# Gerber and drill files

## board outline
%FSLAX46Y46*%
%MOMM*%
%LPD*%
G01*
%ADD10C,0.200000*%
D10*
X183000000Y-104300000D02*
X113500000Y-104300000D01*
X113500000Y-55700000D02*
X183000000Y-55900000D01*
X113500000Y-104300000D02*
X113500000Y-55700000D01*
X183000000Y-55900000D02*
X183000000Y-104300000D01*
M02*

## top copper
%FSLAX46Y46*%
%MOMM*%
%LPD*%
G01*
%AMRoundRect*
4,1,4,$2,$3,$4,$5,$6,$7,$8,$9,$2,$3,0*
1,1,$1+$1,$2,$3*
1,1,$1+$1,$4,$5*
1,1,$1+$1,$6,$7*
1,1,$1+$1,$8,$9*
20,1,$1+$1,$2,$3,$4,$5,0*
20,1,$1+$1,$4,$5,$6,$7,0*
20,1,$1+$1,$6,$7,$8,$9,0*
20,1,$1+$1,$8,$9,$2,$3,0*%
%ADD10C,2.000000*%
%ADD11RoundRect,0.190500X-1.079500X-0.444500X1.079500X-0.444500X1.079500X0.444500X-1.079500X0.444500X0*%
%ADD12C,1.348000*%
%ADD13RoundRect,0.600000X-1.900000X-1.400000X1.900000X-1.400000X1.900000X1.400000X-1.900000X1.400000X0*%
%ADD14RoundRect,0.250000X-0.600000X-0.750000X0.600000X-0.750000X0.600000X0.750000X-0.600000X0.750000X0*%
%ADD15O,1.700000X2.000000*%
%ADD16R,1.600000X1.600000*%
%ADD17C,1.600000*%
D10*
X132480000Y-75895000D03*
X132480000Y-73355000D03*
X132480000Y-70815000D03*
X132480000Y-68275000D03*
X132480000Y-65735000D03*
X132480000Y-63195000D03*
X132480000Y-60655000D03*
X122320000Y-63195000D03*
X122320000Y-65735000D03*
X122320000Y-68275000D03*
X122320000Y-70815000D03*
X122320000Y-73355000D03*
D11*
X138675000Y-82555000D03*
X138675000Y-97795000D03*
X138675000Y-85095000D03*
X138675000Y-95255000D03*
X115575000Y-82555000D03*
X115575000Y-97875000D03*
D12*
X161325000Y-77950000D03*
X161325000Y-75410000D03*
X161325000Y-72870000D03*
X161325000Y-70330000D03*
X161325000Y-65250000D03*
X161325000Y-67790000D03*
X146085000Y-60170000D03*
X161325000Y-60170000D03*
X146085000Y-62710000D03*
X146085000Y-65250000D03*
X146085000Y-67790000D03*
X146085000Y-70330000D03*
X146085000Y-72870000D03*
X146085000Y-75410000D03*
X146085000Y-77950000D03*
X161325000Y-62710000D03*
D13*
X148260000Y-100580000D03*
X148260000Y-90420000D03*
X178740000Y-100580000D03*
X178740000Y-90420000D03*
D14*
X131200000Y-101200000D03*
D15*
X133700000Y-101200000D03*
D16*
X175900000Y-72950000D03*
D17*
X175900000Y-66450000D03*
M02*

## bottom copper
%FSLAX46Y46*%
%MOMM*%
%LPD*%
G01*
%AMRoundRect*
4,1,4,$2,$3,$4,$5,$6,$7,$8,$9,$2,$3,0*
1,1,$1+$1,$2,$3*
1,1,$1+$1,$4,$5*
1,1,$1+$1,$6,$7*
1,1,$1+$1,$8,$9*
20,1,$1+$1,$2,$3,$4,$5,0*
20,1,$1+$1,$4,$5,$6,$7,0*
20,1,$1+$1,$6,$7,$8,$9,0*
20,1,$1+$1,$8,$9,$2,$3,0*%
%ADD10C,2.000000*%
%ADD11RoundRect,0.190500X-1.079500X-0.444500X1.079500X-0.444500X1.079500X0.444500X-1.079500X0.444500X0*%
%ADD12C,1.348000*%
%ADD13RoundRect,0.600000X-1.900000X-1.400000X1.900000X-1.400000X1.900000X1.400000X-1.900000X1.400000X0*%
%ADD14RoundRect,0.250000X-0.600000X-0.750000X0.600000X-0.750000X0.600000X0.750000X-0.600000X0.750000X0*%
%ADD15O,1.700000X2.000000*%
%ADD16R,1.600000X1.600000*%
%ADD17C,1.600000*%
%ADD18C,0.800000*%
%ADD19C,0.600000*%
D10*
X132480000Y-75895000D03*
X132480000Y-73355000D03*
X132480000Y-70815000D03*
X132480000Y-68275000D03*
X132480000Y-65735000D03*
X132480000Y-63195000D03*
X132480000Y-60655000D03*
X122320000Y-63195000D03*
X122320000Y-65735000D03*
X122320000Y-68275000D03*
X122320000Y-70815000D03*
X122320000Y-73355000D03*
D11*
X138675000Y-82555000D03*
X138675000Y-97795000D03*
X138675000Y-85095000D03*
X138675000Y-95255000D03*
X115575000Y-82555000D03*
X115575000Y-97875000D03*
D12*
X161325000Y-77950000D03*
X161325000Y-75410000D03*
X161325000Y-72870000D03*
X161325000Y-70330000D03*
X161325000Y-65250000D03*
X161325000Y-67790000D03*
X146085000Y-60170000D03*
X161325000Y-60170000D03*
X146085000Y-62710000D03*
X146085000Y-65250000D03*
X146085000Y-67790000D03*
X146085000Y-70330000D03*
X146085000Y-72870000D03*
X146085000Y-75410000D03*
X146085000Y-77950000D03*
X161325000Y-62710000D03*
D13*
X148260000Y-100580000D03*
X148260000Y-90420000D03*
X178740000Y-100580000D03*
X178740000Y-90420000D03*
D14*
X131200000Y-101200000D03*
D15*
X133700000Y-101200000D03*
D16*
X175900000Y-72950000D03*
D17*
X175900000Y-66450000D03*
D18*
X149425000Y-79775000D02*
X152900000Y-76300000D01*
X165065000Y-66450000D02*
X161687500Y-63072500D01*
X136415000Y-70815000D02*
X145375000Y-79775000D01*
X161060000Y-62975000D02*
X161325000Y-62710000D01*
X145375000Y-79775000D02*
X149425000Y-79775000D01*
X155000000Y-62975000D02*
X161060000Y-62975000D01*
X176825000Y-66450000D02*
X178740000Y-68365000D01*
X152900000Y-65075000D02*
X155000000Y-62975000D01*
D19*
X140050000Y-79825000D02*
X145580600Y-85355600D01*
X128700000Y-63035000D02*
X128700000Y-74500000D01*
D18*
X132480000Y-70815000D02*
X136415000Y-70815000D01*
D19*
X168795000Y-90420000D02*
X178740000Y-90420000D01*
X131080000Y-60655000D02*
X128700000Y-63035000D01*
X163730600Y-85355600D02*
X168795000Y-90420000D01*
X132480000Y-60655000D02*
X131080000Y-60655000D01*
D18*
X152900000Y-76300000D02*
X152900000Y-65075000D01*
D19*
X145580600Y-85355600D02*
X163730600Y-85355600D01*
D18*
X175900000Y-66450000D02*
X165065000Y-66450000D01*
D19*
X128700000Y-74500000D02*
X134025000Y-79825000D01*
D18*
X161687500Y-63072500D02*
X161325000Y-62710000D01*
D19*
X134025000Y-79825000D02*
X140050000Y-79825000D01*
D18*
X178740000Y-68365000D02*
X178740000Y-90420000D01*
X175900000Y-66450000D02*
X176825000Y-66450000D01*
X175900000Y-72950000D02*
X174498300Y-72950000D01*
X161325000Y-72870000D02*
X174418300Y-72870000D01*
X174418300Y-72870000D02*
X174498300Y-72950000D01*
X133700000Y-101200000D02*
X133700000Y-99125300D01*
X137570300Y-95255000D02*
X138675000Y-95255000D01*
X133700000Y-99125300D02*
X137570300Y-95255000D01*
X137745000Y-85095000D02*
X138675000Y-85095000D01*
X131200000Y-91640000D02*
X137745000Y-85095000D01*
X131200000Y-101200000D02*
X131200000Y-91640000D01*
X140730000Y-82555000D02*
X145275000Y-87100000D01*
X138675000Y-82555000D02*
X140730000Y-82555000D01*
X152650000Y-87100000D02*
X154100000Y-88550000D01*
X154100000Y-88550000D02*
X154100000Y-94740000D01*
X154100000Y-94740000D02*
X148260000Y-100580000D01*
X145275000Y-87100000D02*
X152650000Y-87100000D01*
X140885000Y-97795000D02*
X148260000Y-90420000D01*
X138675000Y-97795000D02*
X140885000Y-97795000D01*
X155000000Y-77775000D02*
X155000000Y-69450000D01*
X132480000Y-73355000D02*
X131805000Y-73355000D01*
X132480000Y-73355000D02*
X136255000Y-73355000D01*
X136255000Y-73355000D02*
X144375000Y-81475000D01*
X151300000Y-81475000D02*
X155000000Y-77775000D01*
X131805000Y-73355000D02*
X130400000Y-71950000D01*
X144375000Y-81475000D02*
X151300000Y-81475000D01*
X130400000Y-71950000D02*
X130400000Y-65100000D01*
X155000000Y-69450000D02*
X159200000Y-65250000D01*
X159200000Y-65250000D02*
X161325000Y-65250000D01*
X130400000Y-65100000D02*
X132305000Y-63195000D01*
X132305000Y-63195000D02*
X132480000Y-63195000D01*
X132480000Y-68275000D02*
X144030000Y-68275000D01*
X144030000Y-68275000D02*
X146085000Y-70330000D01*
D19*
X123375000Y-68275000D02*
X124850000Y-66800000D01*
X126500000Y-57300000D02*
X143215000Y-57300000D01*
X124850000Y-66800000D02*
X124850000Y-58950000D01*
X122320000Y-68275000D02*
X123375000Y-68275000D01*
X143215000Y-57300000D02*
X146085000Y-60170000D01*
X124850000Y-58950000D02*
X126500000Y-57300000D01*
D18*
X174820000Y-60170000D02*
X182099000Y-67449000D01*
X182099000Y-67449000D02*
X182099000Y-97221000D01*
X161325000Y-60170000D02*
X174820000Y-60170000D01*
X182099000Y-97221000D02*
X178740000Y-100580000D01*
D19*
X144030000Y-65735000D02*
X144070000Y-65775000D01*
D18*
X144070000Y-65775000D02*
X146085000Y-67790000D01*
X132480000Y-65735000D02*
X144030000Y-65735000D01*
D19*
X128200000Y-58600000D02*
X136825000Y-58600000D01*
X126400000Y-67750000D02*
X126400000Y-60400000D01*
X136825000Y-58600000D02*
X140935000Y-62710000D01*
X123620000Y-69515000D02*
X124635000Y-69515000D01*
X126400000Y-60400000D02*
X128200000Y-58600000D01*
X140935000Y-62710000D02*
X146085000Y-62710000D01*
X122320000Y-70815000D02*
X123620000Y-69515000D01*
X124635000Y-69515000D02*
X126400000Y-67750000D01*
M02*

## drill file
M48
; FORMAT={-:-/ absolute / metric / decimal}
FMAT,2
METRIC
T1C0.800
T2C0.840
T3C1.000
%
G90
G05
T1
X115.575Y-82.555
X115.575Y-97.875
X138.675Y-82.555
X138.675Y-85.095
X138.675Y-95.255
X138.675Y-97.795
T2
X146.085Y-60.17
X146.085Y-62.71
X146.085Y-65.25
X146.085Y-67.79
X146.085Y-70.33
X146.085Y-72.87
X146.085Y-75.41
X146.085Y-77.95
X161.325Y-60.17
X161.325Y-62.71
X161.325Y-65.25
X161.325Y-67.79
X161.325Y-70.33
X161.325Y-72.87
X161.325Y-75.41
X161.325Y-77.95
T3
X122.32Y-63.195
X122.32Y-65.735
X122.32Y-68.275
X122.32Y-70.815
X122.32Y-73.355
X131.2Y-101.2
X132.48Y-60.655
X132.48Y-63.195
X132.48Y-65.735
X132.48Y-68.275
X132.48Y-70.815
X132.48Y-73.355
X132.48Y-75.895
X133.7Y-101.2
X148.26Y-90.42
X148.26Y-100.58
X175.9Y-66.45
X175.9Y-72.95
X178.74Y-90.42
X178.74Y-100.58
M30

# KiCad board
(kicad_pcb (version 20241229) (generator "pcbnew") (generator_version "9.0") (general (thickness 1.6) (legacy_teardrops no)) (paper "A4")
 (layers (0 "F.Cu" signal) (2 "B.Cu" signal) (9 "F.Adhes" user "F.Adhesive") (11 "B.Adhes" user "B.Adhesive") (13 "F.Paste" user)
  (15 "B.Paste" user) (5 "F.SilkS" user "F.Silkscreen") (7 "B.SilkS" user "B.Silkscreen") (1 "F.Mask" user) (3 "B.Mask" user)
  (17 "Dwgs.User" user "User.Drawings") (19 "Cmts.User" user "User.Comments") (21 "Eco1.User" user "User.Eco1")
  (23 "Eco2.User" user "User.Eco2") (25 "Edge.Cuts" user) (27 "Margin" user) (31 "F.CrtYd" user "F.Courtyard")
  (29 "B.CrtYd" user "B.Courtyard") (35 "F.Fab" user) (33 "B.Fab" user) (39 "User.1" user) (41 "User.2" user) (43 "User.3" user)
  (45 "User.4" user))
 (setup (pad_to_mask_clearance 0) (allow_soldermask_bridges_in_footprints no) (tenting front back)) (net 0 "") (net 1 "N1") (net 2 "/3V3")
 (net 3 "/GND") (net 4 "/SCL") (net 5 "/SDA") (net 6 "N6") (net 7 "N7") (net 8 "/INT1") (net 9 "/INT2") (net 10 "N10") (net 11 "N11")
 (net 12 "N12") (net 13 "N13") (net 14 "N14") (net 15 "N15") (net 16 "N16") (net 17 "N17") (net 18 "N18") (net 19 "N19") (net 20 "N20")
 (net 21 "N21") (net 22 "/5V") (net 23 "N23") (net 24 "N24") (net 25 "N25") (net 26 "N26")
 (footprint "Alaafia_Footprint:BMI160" (layer "F.Cu") (at 127.4 68.275 180)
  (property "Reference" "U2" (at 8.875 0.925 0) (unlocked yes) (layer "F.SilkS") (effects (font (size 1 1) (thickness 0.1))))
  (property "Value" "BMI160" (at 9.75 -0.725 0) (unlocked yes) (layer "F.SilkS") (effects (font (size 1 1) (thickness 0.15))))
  (pad "1" thru_hole circle (at -5.08 -7.62 180) (size 2 2) (drill 1) (layers "*.Cu" "*.Mask") (remove_unused_layers no) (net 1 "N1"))
  (pad "2" thru_hole circle (at -5.08 -5.08 180) (size 2 2) (drill 1) (layers "*.Cu" "*.Mask") (remove_unused_layers no) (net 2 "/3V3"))
  (pad "3" thru_hole circle (at -5.08 -2.54 180) (size 2 2) (drill 1) (layers "*.Cu" "*.Mask") (remove_unused_layers no) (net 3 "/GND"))
  (pad "4" thru_hole circle (at -5.08 0 180) (size 2 2) (drill 1) (layers "*.Cu" "*.Mask") (remove_unused_layers no) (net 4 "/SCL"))
  (pad "5" thru_hole circle (at -5.08 2.54 180) (size 2 2) (drill 1) (layers "*.Cu" "*.Mask") (remove_unused_layers no) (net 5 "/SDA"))
  (pad "6" thru_hole circle (at -5.08 5.08 180) (size 2 2) (drill 1) (layers "*.Cu" "*.Mask") (remove_unused_layers no) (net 2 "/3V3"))
  (pad "7" thru_hole circle (at -5.08 7.62 180) (size 2 2) (drill 1) (layers "*.Cu" "*.Mask") (remove_unused_layers no) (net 3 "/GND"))
  (pad "8" thru_hole circle (at 5.08 5.08 180) (size 2 2) (drill 1) (layers "*.Cu" "*.Mask") (remove_unused_layers no) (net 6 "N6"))
  (pad "9" thru_hole circle (at 5.08 2.54 180) (size 2 2) (drill 1) (layers "*.Cu" "*.Mask") (remove_unused_layers no) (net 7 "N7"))
  (pad "10" thru_hole circle (at 5.08 0 180) (size 2 2) (drill 1) (layers "*.Cu" "*.Mask") (remove_unused_layers no) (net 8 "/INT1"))
  (pad "11" thru_hole circle (at 5.08 -2.54 180) (size 2 2) (drill 1) (layers "*.Cu" "*.Mask") (remove_unused_layers no) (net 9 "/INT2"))
  (pad "12" thru_hole circle (at 5.08 -5.08 180) (size 2 2) (drill 1) (layers "*.Cu" "*.Mask") (remove_unused_layers no) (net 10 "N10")))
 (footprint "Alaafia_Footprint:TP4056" (layer "F.Cu") (at 128.075 90.175)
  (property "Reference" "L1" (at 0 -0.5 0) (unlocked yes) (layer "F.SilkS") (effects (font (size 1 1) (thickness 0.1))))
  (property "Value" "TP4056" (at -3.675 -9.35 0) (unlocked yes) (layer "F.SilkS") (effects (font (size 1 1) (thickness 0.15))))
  (pad "1" thru_hole roundrect (at 10.6 -7.62) (size 2.54 1.27) (drill 0.8) (layers "*.Cu" "*.Mask") (remove_unused_layers no)
   (roundrect_rratio 0.15) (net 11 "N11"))
  (pad "2" thru_hole roundrect (at 10.6 7.62) (size 2.54 1.27) (drill 0.8) (layers "*.Cu" "*.Mask") (remove_unused_layers no)
   (roundrect_rratio 0.15) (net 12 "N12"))
  (pad "3" thru_hole roundrect (at 10.6 -5.08) (size 2.54 1.27) (drill 0.8) (layers "*.Cu" "*.Mask") (remove_unused_layers no)
   (roundrect_rratio 0.15) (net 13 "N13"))
  (pad "4" thru_hole roundrect (at 10.6 5.08) (size 2.54 1.27) (drill 0.8) (layers "*.Cu" "*.Mask") (remove_unused_layers no)
   (roundrect_rratio 0.15) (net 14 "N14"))
  (pad "5" thru_hole roundrect (at -12.5 -7.62) (size 2.54 1.27) (drill 0.8) (layers "*.Cu" "*.Mask") (remove_unused_layers no)
   (roundrect_rratio 0.15) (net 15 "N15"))
  (pad "6" thru_hole roundrect (at -12.5 7.7) (size 2.54 1.27) (drill 0.8) (layers "*.Cu" "*.Mask") (remove_unused_layers no)
   (roundrect_rratio 0.15) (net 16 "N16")))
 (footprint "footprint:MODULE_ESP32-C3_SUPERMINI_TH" (layer "F.Cu") (at 153.705 70.07)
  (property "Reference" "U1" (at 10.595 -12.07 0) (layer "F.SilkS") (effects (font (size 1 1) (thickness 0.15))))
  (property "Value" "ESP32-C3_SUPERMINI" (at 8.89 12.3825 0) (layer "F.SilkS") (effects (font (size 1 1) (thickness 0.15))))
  (pad "0" thru_hole circle (at 7.62 7.88) (size 1.348 1.348) (drill 0.84) (layers "*.Cu" "*.Mask") (remove_unused_layers no) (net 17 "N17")
   (solder_mask_margin 0.102))
  (pad "1" thru_hole circle (at 7.62 5.34) (size 1.348 1.348) (drill 0.84) (layers "*.Cu" "*.Mask") (remove_unused_layers no) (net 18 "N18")
   (solder_mask_margin 0.102))
  (pad "2" thru_hole circle (at 7.62 2.8) (size 1.348 1.348) (drill 0.84) (layers "*.Cu" "*.Mask") (remove_unused_layers no) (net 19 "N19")
   (solder_mask_margin 0.102))
  (pad "3" thru_hole circle (at 7.62 0.26) (size 1.348 1.348) (drill 0.84) (layers "*.Cu" "*.Mask") (remove_unused_layers no) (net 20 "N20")
   (solder_mask_margin 0.102))
  (pad "3.3" thru_hole circle (at 7.62 -4.82) (size 1.348 1.348) (drill 0.84) (layers "*.Cu" "*.Mask") (remove_unused_layers no)
   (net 2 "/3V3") (solder_mask_margin 0.102))
  (pad "4" thru_hole circle (at 7.62 -2.28) (size 1.348 1.348) (drill 0.84) (layers "*.Cu" "*.Mask") (remove_unused_layers no)
   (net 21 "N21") (solder_mask_margin 0.102))
  (pad "5" thru_hole circle (at -7.62 -9.9) (size 1.348 1.348) (drill 0.84) (layers "*.Cu" "*.Mask") (remove_unused_layers no)
   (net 8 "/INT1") (solder_mask_margin 0.102))
  (pad "5V" thru_hole circle (at 7.62 -9.9) (size 1.348 1.348) (drill 0.84) (layers "*.Cu" "*.Mask") (remove_unused_layers no)
   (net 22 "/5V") (solder_mask_margin 0.102))
  (pad "6" thru_hole circle (at -7.62 -7.36) (size 1.348 1.348) (drill 0.84) (layers "*.Cu" "*.Mask") (remove_unused_layers no)
   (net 9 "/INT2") (solder_mask_margin 0.102))
  (pad "7" thru_hole circle (at -7.62 -4.82) (size 1.348 1.348) (drill 0.84) (layers "*.Cu" "*.Mask") (remove_unused_layers no)
   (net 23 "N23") (solder_mask_margin 0.102))
  (pad "8" thru_hole circle (at -7.62 -2.28) (size 1.348 1.348) (drill 0.84) (layers "*.Cu" "*.Mask") (remove_unused_layers no)
   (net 5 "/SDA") (solder_mask_margin 0.102))
  (pad "9" thru_hole circle (at -7.62 0.26) (size 1.348 1.348) (drill 0.84) (layers "*.Cu" "*.Mask") (remove_unused_layers no)
   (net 4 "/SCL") (solder_mask_margin 0.102))
  (pad "10" thru_hole circle (at -7.62 2.8) (size 1.348 1.348) (drill 0.84) (layers "*.Cu" "*.Mask") (remove_unused_layers no)
   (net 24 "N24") (solder_mask_margin 0.102))
  (pad "20" thru_hole circle (at -7.62 5.34) (size 1.348 1.348) (drill 0.84) (layers "*.Cu" "*.Mask") (remove_unused_layers no)
   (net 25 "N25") (solder_mask_margin 0.102))
  (pad "21" thru_hole circle (at -7.62 7.88) (size 1.348 1.348) (drill 0.84) (layers "*.Cu" "*.Mask") (remove_unused_layers no)
   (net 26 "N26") (solder_mask_margin 0.102))
  (pad "G" thru_hole circle (at 7.62 -7.36) (size 1.348 1.348) (drill 0.84) (layers "*.Cu" "*.Mask") (remove_unused_layers no)
   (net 3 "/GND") (solder_mask_margin 0.102)))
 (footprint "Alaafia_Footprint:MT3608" (layer "F.Cu") (at 163.5 95.5)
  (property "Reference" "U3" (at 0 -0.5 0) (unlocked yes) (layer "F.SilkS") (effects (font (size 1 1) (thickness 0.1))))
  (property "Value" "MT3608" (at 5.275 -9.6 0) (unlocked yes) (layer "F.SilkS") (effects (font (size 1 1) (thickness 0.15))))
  (pad "1" thru_hole roundrect (at -15.24 5.08) (size 5 4) (drill 1) (layers "*.Cu" "*.Mask") (remove_unused_layers no)
   (roundrect_rratio 0.15) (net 11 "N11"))
  (pad "2" thru_hole roundrect (at -15.24 -5.08) (size 5 4) (drill 1) (layers "*.Cu" "*.Mask") (remove_unused_layers no)
   (roundrect_rratio 0.15) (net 12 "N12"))
  (pad "3" thru_hole roundrect (at 15.24 5.08) (size 5 4) (drill 1) (layers "*.Cu" "*.Mask") (remove_unused_layers no)
   (roundrect_rratio 0.15) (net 22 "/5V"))
  (pad "4" thru_hole roundrect (at 15.24 -5.08) (size 5 4) (drill 1) (layers "*.Cu" "*.Mask") (remove_unused_layers no)
   (roundrect_rratio 0.15) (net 3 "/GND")))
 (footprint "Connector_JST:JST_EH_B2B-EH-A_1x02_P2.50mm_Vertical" (layer "F.Cu") (at 131.2 101.2)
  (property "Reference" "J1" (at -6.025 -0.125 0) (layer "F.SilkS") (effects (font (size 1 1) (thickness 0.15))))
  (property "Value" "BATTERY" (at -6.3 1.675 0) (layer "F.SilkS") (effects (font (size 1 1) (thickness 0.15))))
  (pad "1" thru_hole roundrect (at 0 0) (size 1.7 2) (drill 1) (layers "*.Cu" "*.Mask") (remove_unused_layers no)
   (roundrect_rratio 0.147059) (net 13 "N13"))
  (pad "2" thru_hole oval (at 2.5 0) (size 1.7 2) (drill 1) (layers "*.Cu" "*.Mask") (remove_unused_layers no) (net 14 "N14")))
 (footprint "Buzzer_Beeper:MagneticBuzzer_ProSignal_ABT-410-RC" (layer "F.Cu") (at 175.9 72.95 90)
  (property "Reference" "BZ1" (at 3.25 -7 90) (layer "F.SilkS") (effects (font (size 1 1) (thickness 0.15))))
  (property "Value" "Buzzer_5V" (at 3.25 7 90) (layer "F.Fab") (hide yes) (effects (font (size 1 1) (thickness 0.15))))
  (pad "1" thru_hole rect (at 0 0 90) (size 1.6 1.6) (drill 1) (layers "*.Cu" "*.Mask") (remove_unused_layers no) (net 19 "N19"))
  (pad "2" thru_hole circle (at 6.5 0 90) (size 1.6 1.6) (drill 1) (layers "*.Cu" "*.Mask") (remove_unused_layers no) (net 3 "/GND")))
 (gr_line (start 183 104.3) (end 113.5 104.3) (stroke (width 0.2) (type solid)) (layer "Edge.Cuts"))
 (gr_line (start 113.5 55.7) (end 183 55.9) (stroke (width 0.2) (type solid)) (layer "Edge.Cuts"))
 (gr_line (start 113.5 104.3) (end 113.5 55.7) (stroke (width 0.2) (type solid)) (layer "Edge.Cuts"))
 (gr_line (start 183 55.9) (end 183 104.3) (stroke (width 0.2) (type solid)) (layer "Edge.Cuts"))
 (segment (start 149.425 79.775) (end 152.9 76.3) (width 0.8) (layer "B.Cu") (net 3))
 (segment (start 165.065 66.45) (end 161.6875 63.0725) (width 0.8) (layer "B.Cu") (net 3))
 (segment (start 136.415 70.815) (end 145.375 79.775) (width 0.8) (layer "B.Cu") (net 3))
 (segment (start 161.06 62.975) (end 161.325 62.71) (width 0.8) (layer "B.Cu") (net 3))
 (segment (start 145.375 79.775) (end 149.425 79.775) (width 0.8) (layer "B.Cu") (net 3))
 (segment (start 155 62.975) (end 161.06 62.975) (width 0.8) (layer "B.Cu") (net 3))
 (segment (start 176.825 66.45) (end 178.74 68.365) (width 0.8) (layer "B.Cu") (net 3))
 (segment (start 152.9 65.075) (end 155 62.975) (width 0.8) (layer "B.Cu") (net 3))
 (segment (start 140.05 79.825) (end 145.5806 85.3556) (width 0.6) (layer "B.Cu") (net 3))
 (segment (start 128.7 63.035) (end 128.7 74.5) (width 0.6) (layer "B.Cu") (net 3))
 (segment (start 132.48 70.815) (end 136.415 70.815) (width 0.8) (layer "B.Cu") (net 3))
 (segment (start 168.795 90.42) (end 178.74 90.42) (width 0.6) (layer "B.Cu") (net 3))
 (segment (start 131.08 60.655) (end 128.7 63.035) (width 0.6) (layer "B.Cu") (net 3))
 (segment (start 163.7306 85.3556) (end 168.795 90.42) (width 0.6) (layer "B.Cu") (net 3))
 (segment (start 132.48 60.655) (end 131.08 60.655) (width 0.6) (layer "B.Cu") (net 3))
 (segment (start 152.9 76.3) (end 152.9 65.075) (width 0.8) (layer "B.Cu") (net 3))
 (segment (start 145.5806 85.3556) (end 163.7306 85.3556) (width 0.6) (layer "B.Cu") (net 3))
 (segment (start 175.9 66.45) (end 165.065 66.45) (width 0.8) (layer "B.Cu") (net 3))
 (segment (start 128.7 74.5) (end 134.025 79.825) (width 0.6) (layer "B.Cu") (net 3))
 (segment (start 161.6875 63.0725) (end 161.325 62.71) (width 0.8) (layer "B.Cu") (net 3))
 (segment (start 134.025 79.825) (end 140.05 79.825) (width 0.6) (layer "B.Cu") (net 3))
 (segment (start 178.74 68.365) (end 178.74 90.42) (width 0.8) (layer "B.Cu") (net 3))
 (segment (start 175.9 66.45) (end 176.825 66.45) (width 0.8) (layer "B.Cu") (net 3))
 (segment (start 175.9 72.95) (end 174.4983 72.95) (width 0.8) (layer "B.Cu") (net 19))
 (segment (start 161.325 72.87) (end 174.4183 72.87) (width 0.8) (layer "B.Cu") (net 19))
 (segment (start 174.4183 72.87) (end 174.4983 72.95) (width 0.8) (layer "B.Cu") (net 19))
 (segment (start 133.7 101.2) (end 133.7 99.1253) (width 0.8) (layer "B.Cu") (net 14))
 (segment (start 137.5703 95.255) (end 138.675 95.255) (width 0.8) (layer "B.Cu") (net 14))
 (segment (start 133.7 99.1253) (end 137.5703 95.255) (width 0.8) (layer "B.Cu") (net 14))
 (segment (start 137.745 85.095) (end 138.675 85.095) (width 0.8) (layer "B.Cu") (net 13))
 (segment (start 131.2 91.64) (end 137.745 85.095) (width 0.8) (layer "B.Cu") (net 13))
 (segment (start 131.2 101.2) (end 131.2 91.64) (width 0.8) (layer "B.Cu") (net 13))
 (segment (start 140.73 82.555) (end 145.275 87.1) (width 0.8) (layer "B.Cu") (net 11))
 (segment (start 138.675 82.555) (end 140.73 82.555) (width 0.8) (layer "B.Cu") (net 11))
 (segment (start 152.65 87.1) (end 154.1 88.55) (width 0.8) (layer "B.Cu") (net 11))
 (segment (start 154.1 88.55) (end 154.1 94.74) (width 0.8) (layer "B.Cu") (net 11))
 (segment (start 154.1 94.74) (end 148.26 100.58) (width 0.8) (layer "B.Cu") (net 11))
 (segment (start 145.275 87.1) (end 152.65 87.1) (width 0.8) (layer "B.Cu") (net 11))
 (segment (start 140.885 97.795) (end 148.26 90.42) (width 0.8) (layer "B.Cu") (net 12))
 (segment (start 138.675 97.795) (end 140.885 97.795) (width 0.8) (layer "B.Cu") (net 12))
 (segment (start 155 77.775) (end 155 69.45) (width 0.8) (layer "B.Cu") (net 2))
 (segment (start 132.48 73.355) (end 131.805 73.355) (width 0.8) (layer "B.Cu") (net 2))
 (segment (start 132.48 73.355) (end 136.255 73.355) (width 0.8) (layer "B.Cu") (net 2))
 (segment (start 136.255 73.355) (end 144.375 81.475) (width 0.8) (layer "B.Cu") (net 2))
 (segment (start 151.3 81.475) (end 155 77.775) (width 0.8) (layer "B.Cu") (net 2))
 (segment (start 131.805 73.355) (end 130.4 71.95) (width 0.8) (layer "B.Cu") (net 2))
 (segment (start 144.375 81.475) (end 151.3 81.475) (width 0.8) (layer "B.Cu") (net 2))
 (segment (start 130.4 71.95) (end 130.4 65.1) (width 0.8) (layer "B.Cu") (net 2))
 (segment (start 155 69.45) (end 159.2 65.25) (width 0.8) (layer "B.Cu") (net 2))
 (segment (start 159.2 65.25) (end 161.325 65.25) (width 0.8) (layer "B.Cu") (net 2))
 (segment (start 130.4 65.1) (end 132.305 63.195) (width 0.8) (layer "B.Cu") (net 2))
 (segment (start 132.305 63.195) (end 132.48 63.195) (width 0.8) (layer "B.Cu") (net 2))
 (segment (start 132.48 68.275) (end 144.03 68.275) (width 0.8) (layer "B.Cu") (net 4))
 (segment (start 144.03 68.275) (end 146.085 70.33) (width 0.8) (layer "B.Cu") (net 4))
 (segment (start 123.375 68.275) (end 124.85 66.8) (width 0.6) (layer "B.Cu") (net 8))
 (segment (start 126.5 57.3) (end 143.215 57.3) (width 0.6) (layer "B.Cu") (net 8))
 (segment (start 124.85 66.8) (end 124.85 58.95) (width 0.6) (layer "B.Cu") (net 8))
 (segment (start 122.32 68.275) (end 123.375 68.275) (width 0.6) (layer "B.Cu") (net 8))
 (segment (start 143.215 57.3) (end 146.085 60.17) (width 0.6) (layer "B.Cu") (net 8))
 (segment (start 124.85 58.95) (end 126.5 57.3) (width 0.6) (layer "B.Cu") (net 8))
 (segment (start 174.82 60.17) (end 182.099 67.449) (width 0.8) (layer "B.Cu") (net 22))
 (segment (start 182.099 67.449) (end 182.099 97.221) (width 0.8) (layer "B.Cu") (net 22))
 (segment (start 161.325 60.17) (end 174.82 60.17) (width 0.8) (layer "B.Cu") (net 22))
 (segment (start 182.099 97.221) (end 178.74 100.58) (width 0.8) (layer "B.Cu") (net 22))
 (segment (start 144.03 65.735) (end 144.07 65.775) (width 0.6) (layer "B.Cu") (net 5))
 (segment (start 144.07 65.775) (end 146.085 67.79) (width 0.8) (layer "B.Cu") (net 5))
 (segment (start 132.48 65.735) (end 144.03 65.735) (width 0.8) (layer "B.Cu") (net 5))
 (segment (start 128.2 58.6) (end 136.825 58.6) (width 0.6) (layer "B.Cu") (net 9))
 (segment (start 126.4 67.75) (end 126.4 60.4) (width 0.6) (layer "B.Cu") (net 9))
 (segment (start 136.825 58.6) (end 140.935 62.71) (width 0.6) (layer "B.Cu") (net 9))
 (segment (start 123.62 69.515) (end 124.635 69.515) (width 0.6) (layer "B.Cu") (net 9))
 (segment (start 126.4 60.4) (end 128.2 58.6) (width 0.6) (layer "B.Cu") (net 9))
 (segment (start 140.935 62.71) (end 146.085 62.71) (width 0.6) (layer "B.Cu") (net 9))
 (segment (start 122.32 70.815) (end 123.62 69.515) (width 0.6) (layer "B.Cu") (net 9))
 (segment (start 124.635 69.515) (end 126.4 67.75) (width 0.6) (layer "B.Cu") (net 9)))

